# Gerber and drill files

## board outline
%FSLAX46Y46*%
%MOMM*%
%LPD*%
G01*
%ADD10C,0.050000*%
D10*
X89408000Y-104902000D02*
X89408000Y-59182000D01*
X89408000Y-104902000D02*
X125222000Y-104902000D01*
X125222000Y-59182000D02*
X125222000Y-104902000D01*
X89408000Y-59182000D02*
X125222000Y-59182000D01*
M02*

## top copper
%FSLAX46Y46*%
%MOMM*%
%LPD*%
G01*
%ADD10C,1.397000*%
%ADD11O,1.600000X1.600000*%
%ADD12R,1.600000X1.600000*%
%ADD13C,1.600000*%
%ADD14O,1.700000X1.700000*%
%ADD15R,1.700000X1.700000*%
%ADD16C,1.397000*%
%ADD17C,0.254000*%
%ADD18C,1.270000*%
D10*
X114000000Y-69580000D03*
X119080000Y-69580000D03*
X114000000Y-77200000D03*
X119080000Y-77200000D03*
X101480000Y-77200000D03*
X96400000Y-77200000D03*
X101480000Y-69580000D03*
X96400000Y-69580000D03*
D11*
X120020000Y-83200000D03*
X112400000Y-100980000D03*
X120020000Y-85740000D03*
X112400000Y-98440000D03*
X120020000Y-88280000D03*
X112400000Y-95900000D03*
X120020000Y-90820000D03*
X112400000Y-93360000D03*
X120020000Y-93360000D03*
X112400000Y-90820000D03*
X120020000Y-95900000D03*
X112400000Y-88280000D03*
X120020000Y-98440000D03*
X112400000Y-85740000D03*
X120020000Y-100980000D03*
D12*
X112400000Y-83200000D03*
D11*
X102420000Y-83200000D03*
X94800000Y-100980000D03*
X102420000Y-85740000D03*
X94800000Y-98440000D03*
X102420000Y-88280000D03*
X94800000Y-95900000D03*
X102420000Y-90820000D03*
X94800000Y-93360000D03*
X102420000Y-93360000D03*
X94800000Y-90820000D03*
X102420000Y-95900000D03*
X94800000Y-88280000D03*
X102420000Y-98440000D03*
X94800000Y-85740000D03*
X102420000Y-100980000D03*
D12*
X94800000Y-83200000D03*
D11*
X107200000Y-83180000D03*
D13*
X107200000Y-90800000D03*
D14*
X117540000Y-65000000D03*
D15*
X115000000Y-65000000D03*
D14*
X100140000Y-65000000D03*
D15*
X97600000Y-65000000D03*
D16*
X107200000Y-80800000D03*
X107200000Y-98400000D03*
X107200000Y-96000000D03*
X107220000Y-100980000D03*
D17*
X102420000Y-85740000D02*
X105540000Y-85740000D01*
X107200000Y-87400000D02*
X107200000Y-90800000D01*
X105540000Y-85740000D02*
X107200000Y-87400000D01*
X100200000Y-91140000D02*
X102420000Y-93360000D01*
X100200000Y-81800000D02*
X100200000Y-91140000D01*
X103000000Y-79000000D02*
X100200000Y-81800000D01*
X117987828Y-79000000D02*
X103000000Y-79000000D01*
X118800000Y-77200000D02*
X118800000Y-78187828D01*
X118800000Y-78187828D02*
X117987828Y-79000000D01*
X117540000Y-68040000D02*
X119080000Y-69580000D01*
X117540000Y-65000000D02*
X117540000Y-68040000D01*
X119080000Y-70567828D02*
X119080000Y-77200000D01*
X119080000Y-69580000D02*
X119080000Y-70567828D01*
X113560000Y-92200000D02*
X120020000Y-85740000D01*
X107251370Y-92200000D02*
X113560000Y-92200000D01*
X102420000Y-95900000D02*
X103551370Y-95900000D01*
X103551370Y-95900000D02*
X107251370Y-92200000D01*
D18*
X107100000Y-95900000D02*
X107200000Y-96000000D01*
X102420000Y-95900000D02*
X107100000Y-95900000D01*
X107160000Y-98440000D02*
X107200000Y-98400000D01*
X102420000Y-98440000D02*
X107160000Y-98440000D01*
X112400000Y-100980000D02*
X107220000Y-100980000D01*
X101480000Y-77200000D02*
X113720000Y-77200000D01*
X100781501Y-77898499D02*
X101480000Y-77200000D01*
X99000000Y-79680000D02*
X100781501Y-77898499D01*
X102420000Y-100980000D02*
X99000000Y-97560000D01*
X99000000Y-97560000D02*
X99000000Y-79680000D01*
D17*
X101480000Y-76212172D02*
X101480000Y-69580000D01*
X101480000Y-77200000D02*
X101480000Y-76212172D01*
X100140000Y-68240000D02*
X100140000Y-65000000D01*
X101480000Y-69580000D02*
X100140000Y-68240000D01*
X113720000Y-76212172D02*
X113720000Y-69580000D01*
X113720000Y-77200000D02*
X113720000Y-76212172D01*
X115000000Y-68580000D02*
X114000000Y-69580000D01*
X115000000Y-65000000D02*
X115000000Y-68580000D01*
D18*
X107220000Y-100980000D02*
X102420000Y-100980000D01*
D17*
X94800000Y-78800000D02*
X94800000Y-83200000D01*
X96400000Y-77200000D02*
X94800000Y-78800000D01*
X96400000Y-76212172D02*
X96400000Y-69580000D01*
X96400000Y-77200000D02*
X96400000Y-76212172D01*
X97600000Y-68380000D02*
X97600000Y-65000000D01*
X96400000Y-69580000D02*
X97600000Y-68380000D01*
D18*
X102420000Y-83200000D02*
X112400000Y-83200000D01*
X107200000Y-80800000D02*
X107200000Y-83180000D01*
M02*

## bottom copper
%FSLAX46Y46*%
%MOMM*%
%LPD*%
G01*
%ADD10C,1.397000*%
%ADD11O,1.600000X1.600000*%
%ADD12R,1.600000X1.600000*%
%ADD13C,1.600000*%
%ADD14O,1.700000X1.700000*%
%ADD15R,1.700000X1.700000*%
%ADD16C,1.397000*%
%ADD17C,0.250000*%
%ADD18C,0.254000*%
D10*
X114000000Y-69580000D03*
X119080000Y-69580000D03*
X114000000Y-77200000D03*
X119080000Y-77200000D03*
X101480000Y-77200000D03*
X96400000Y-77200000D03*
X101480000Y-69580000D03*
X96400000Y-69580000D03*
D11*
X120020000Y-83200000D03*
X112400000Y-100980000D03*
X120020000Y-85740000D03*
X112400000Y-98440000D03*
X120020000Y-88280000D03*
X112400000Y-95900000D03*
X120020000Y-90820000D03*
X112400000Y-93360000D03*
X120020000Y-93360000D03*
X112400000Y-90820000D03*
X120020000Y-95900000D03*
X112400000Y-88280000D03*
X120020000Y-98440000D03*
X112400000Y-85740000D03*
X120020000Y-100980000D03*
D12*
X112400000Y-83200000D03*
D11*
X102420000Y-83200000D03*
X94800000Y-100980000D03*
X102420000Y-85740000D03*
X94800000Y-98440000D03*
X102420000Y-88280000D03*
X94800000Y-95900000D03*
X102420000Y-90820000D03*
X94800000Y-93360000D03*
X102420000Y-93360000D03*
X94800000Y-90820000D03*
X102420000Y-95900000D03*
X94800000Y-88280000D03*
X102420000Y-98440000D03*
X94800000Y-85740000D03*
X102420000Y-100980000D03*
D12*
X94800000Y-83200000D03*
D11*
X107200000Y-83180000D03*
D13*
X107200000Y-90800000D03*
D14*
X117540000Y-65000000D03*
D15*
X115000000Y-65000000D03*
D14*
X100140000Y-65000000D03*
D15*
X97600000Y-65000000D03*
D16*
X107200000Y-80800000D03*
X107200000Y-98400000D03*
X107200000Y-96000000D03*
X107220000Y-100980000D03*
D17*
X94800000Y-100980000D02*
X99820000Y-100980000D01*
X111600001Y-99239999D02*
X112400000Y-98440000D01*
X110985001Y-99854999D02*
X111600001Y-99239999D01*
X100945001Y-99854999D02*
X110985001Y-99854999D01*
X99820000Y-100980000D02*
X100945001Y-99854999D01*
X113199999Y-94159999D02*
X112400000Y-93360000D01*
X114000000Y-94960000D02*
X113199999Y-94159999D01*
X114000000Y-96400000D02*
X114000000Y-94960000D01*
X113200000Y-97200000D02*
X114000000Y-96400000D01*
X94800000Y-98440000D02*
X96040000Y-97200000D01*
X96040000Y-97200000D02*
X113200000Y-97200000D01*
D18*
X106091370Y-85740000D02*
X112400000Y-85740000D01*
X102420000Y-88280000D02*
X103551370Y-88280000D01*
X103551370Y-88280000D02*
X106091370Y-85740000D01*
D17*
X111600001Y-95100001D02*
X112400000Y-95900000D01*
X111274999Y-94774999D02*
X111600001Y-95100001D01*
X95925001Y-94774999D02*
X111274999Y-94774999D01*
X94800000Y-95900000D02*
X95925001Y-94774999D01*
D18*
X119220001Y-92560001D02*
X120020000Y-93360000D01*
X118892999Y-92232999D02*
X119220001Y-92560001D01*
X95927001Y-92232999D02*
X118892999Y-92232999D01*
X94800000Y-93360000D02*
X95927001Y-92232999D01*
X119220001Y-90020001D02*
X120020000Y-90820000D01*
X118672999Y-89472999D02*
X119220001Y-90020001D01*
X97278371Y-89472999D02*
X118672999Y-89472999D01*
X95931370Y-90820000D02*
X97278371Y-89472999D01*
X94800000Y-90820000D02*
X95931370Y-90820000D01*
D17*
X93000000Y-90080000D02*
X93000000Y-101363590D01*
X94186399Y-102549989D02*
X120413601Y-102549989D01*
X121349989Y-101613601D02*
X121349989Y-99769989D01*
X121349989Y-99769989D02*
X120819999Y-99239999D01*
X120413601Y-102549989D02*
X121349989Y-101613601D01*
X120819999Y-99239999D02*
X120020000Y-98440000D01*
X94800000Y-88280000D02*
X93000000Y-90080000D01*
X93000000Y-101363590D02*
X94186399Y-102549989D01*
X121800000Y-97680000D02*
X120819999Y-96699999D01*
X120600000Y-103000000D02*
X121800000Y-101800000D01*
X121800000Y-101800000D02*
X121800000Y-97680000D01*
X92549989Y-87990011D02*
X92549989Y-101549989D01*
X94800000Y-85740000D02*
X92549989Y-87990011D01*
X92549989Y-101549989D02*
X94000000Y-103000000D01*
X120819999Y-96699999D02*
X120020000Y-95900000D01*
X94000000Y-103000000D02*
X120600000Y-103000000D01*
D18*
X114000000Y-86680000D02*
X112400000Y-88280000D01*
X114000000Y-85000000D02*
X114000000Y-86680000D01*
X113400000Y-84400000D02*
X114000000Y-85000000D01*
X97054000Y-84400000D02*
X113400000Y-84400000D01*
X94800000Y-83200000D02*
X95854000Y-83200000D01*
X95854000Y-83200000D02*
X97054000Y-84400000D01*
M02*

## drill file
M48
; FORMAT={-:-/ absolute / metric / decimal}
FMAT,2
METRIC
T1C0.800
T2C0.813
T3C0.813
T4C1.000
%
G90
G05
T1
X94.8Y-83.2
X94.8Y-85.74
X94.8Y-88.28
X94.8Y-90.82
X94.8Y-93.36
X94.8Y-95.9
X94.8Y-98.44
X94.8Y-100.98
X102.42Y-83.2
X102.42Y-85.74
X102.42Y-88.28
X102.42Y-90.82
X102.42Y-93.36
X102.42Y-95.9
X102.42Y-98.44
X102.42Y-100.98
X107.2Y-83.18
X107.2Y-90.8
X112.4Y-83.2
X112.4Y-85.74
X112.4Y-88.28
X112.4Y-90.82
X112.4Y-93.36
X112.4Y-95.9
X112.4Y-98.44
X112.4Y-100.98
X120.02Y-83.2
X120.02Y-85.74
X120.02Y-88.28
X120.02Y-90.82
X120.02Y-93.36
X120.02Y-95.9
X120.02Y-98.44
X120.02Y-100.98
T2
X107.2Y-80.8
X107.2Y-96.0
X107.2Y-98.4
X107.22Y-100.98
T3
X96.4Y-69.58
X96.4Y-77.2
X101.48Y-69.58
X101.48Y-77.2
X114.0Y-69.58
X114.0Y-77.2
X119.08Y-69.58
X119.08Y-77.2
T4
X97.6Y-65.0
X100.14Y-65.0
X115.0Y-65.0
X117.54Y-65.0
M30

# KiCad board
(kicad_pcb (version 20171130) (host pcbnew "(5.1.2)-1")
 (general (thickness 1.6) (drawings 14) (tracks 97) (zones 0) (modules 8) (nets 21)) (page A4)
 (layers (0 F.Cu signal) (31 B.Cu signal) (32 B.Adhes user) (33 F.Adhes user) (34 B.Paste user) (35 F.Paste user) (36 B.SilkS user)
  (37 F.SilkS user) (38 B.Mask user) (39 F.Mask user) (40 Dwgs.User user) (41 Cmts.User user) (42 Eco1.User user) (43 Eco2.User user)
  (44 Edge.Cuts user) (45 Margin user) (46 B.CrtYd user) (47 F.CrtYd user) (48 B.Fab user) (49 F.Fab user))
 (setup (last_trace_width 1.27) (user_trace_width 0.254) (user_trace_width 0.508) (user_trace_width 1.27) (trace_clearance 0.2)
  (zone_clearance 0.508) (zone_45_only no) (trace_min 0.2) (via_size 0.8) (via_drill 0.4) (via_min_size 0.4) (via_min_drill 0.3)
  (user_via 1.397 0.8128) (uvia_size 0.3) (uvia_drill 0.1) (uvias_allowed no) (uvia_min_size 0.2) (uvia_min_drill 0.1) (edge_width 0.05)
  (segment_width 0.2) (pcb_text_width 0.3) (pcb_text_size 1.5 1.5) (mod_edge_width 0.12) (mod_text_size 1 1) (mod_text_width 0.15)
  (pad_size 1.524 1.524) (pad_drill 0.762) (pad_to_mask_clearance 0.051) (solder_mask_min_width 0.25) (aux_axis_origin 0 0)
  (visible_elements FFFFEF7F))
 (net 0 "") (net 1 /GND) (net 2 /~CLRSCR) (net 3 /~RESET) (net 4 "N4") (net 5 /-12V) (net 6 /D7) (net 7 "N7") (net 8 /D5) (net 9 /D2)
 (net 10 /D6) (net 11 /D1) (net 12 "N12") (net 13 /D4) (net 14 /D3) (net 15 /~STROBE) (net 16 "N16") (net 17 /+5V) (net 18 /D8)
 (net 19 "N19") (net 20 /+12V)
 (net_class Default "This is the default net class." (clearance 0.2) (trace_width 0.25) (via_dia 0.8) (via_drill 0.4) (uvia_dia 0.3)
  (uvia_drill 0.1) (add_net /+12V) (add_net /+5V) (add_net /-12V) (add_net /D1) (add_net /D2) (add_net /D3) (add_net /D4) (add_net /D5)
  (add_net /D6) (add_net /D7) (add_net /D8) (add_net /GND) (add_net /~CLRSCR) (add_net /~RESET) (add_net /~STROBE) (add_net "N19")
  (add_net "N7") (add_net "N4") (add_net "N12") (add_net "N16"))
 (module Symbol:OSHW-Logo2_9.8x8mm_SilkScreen (layer F.Cu) (at 107.2388 71.1454 90)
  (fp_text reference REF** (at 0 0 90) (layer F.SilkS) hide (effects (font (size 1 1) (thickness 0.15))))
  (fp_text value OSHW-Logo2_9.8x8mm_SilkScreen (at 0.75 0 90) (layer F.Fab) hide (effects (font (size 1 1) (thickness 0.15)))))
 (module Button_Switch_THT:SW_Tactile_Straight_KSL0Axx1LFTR (layer F.Cu) (at 114 77.2 90)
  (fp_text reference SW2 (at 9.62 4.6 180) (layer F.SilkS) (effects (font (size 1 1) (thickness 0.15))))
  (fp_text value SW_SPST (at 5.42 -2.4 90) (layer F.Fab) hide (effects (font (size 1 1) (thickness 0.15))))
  (pad 1 thru_hole circle (at 7.62 0 90) (size 1.397 1.397) (drill 0.8128) (layers *.Cu *.Mask) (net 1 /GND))
  (pad 2 thru_hole circle (at 7.62 5.08 90) (size 1.397 1.397) (drill 0.8128) (layers *.Cu *.Mask) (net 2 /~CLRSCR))
  (pad 1 thru_hole circle (at 0 0 90) (size 1.397 1.397) (drill 0.8128) (layers *.Cu *.Mask) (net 1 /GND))
  (pad 2 thru_hole circle (at 0 5.08 90) (size 1.397 1.397) (drill 0.8128) (layers *.Cu *.Mask) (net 2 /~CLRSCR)))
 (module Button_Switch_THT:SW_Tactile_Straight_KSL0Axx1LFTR (layer F.Cu) (at 96.4 77.2 90)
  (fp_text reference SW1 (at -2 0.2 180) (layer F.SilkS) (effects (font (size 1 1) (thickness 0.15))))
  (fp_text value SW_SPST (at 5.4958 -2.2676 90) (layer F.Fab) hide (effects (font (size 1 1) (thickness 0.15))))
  (pad 2 thru_hole circle (at 0 5.08 90) (size 1.397 1.397) (drill 0.8128) (layers *.Cu *.Mask) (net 1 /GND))
  (pad 1 thru_hole circle (at 0 0 90) (size 1.397 1.397) (drill 0.8128) (layers *.Cu *.Mask) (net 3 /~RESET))
  (pad 2 thru_hole circle (at 7.62 5.08 90) (size 1.397 1.397) (drill 0.8128) (layers *.Cu *.Mask) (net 1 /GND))
  (pad 1 thru_hole circle (at 7.62 0 90) (size 1.397 1.397) (drill 0.8128) (layers *.Cu *.Mask) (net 3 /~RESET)))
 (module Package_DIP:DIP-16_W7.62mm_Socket (layer F.Cu) (at 112.4 83.2)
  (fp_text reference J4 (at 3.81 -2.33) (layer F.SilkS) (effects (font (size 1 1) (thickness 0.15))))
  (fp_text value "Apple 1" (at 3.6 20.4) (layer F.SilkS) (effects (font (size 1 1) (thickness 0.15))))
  (pad 16 thru_hole oval (at 7.62 0) (size 1.6 1.6) (drill 0.8) (layers *.Cu *.Mask) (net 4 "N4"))
  (pad 8 thru_hole oval (at 0 17.78) (size 1.6 1.6) (drill 0.8) (layers *.Cu *.Mask) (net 1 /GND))
  (pad 15 thru_hole oval (at 7.62 2.54) (size 1.6 1.6) (drill 0.8) (layers *.Cu *.Mask) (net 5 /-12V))
  (pad 7 thru_hole oval (at 0 15.24) (size 1.6 1.6) (drill 0.8) (layers *.Cu *.Mask) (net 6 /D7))
  (pad 14 thru_hole oval (at 7.62 5.08) (size 1.6 1.6) (drill 0.8) (layers *.Cu *.Mask) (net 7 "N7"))
  (pad 6 thru_hole oval (at 0 12.7) (size 1.6 1.6) (drill 0.8) (layers *.Cu *.Mask) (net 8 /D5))
  (pad 13 thru_hole oval (at 7.62 7.62) (size 1.6 1.6) (drill 0.8) (layers *.Cu *.Mask) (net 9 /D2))
  (pad 5 thru_hole oval (at 0 10.16) (size 1.6 1.6) (drill 0.8) (layers *.Cu *.Mask) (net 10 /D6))
  (pad 12 thru_hole oval (at 7.62 10.16) (size 1.6 1.6) (drill 0.8) (layers *.Cu *.Mask) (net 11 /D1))
  (pad 4 thru_hole oval (at 0 7.62) (size 1.6 1.6) (drill 0.8) (layers *.Cu *.Mask) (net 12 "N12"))
  (pad 11 thru_hole oval (at 7.62 12.7) (size 1.6 1.6) (drill 0.8) (layers *.Cu *.Mask) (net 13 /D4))
  (pad 3 thru_hole oval (at 0 5.08) (size 1.6 1.6) (drill 0.8) (layers *.Cu *.Mask) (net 3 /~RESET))
  (pad 10 thru_hole oval (at 7.62 15.24) (size 1.6 1.6) (drill 0.8) (layers *.Cu *.Mask) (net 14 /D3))
  (pad 2 thru_hole oval (at 0 2.54) (size 1.6 1.6) (drill 0.8) (layers *.Cu *.Mask) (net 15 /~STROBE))
  (pad 9 thru_hole oval (at 7.62 17.78) (size 1.6 1.6) (drill 0.8) (layers *.Cu *.Mask) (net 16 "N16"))
  (pad 1 thru_hole rect (at 0 0) (size 1.6 1.6) (drill 0.8) (layers *.Cu *.Mask) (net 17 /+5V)))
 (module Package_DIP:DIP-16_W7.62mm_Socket (layer F.Cu) (at 94.8 83.2)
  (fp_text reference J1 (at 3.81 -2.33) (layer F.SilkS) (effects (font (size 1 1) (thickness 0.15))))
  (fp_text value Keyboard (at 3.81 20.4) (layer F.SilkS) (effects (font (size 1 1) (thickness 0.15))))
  (pad 16 thru_hole oval (at 7.62 0) (size 1.6 1.6) (drill 0.8) (layers *.Cu *.Mask) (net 17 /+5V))
  (pad 8 thru_hole oval (at 0 17.78) (size 1.6 1.6) (drill 0.8) (layers *.Cu *.Mask) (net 6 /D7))
  (pad 15 thru_hole oval (at 7.62 2.54) (size 1.6 1.6) (drill 0.8) (layers *.Cu *.Mask) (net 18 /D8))
  (pad 7 thru_hole oval (at 0 15.24) (size 1.6 1.6) (drill 0.8) (layers *.Cu *.Mask) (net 10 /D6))
  (pad 14 thru_hole oval (at 7.62 5.08) (size 1.6 1.6) (drill 0.8) (layers *.Cu *.Mask) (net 15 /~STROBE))
  (pad 6 thru_hole oval (at 0 12.7) (size 1.6 1.6) (drill 0.8) (layers *.Cu *.Mask) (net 8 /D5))
  (pad 13 thru_hole oval (at 7.62 7.62) (size 1.6 1.6) (drill 0.8) (layers *.Cu *.Mask) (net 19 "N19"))
  (pad 5 thru_hole oval (at 0 10.16) (size 1.6 1.6) (drill 0.8) (layers *.Cu *.Mask) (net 11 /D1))
  (pad 12 thru_hole oval (at 7.62 10.16) (size 1.6 1.6) (drill 0.8) (layers *.Cu *.Mask) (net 2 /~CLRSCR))
  (pad 4 thru_hole oval (at 0 7.62) (size 1.6 1.6) (drill 0.8) (layers *.Cu *.Mask) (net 9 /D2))
  (pad 11 thru_hole oval (at 7.62 12.7) (size 1.6 1.6) (drill 0.8) (layers *.Cu *.Mask) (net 5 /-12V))
  (pad 3 thru_hole oval (at 0 5.08) (size 1.6 1.6) (drill 0.8) (layers *.Cu *.Mask) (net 14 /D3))
  (pad 10 thru_hole oval (at 7.62 15.24) (size 1.6 1.6) (drill 0.8) (layers *.Cu *.Mask) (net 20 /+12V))
  (pad 2 thru_hole oval (at 0 2.54) (size 1.6 1.6) (drill 0.8) (layers *.Cu *.Mask) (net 13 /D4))
  (pad 9 thru_hole oval (at 7.62 17.78) (size 1.6 1.6) (drill 0.8) (layers *.Cu *.Mask) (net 1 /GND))
  (pad 1 thru_hole rect (at 0 0) (size 1.6 1.6) (drill 0.8) (layers *.Cu *.Mask) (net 3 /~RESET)))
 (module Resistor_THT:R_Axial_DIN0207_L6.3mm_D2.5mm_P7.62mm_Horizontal (layer F.Cu) (at 107.2 90.8 90)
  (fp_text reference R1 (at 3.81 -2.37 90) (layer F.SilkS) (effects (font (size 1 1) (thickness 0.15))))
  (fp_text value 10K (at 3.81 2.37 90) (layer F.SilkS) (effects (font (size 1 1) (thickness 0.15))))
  (pad 2 thru_hole oval (at 7.62 0 90) (size 1.6 1.6) (drill 0.8) (layers *.Cu *.Mask) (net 17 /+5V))
  (pad 1 thru_hole circle (at 0 0 90) (size 1.6 1.6) (drill 0.8) (layers *.Cu *.Mask) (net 18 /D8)))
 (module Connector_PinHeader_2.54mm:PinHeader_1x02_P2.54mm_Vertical (layer F.Cu) (at 115 65 90)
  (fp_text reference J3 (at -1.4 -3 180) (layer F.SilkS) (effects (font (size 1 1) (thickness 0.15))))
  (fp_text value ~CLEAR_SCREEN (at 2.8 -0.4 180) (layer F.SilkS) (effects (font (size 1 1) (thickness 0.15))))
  (pad 2 thru_hole oval (at 0 2.54 90) (size 1.7 1.7) (drill 1) (layers *.Cu *.Mask) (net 2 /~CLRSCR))
  (pad 1 thru_hole rect (at 0 0 90) (size 1.7 1.7) (drill 1) (layers *.Cu *.Mask) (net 1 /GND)))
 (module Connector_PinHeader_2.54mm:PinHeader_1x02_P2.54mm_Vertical (layer F.Cu) (at 97.6 65 90)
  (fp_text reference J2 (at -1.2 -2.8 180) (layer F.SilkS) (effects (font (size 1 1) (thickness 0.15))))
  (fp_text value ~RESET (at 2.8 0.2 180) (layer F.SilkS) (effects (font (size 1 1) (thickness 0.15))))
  (pad 2 thru_hole oval (at 0 2.54 90) (size 1.7 1.7) (drill 1) (layers *.Cu *.Mask) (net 1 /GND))
  (pad 1 thru_hole rect (at 0 0 90) (size 1.7 1.7) (drill 1) (layers *.Cu *.Mask) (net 3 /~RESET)))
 (gr_line (start 89.408 104.902) (end 89.408 59.182) (layer Edge.Cuts) (width 0.05))
 (gr_line (start 89.408 104.902) (end 125.222 104.902) (layer Edge.Cuts) (width 0.05))
 (gr_line (start 125.222 59.182) (end 125.222 104.902) (layer Edge.Cuts) (width 0.05))
 (gr_line (start 89.408 59.182) (end 125.222 59.182) (layer Edge.Cuts) (width 0.05))
 (via (at 107.2 80.8) (size 1.397) (drill 0.8128) (layers F.Cu B.Cu) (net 17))
 (via (at 107.2 98.4) (size 1.397) (drill 0.8128) (layers F.Cu B.Cu) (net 20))
 (via (at 107.2 96) (size 1.397) (drill 0.8128) (layers F.Cu B.Cu) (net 5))
 (segment (start 94.8 100.98) (end 99.82 100.98) (width 0.25) (layer B.Cu) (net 6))
 (segment (start 111.600001 99.239999) (end 112.4 98.44) (width 0.25) (layer B.Cu) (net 6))
 (segment (start 110.985001 99.854999) (end 111.600001 99.239999) (width 0.25) (layer B.Cu) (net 6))
 (segment (start 100.945001 99.854999) (end 110.985001 99.854999) (width 0.25) (layer B.Cu) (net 6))
 (segment (start 99.82 100.98) (end 100.945001 99.854999) (width 0.25) (layer B.Cu) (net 6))
 (segment (start 102.42 85.74) (end 105.54 85.74) (width 0.254) (layer F.Cu) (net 18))
 (segment (start 107.2 87.4) (end 107.2 90.8) (width 0.254) (layer F.Cu) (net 18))
 (segment (start 105.54 85.74) (end 107.2 87.4) (width 0.254) (layer F.Cu) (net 18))
 (segment (start 113.199999 94.159999) (end 112.4 93.36) (width 0.25) (layer B.Cu) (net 10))
 (segment (start 114 94.96) (end 113.199999 94.159999) (width 0.25) (layer B.Cu) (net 10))
 (segment (start 114 96.4) (end 114 94.96) (width 0.25) (layer B.Cu) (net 10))
 (segment (start 113.2 97.2) (end 114 96.4) (width 0.25) (layer B.Cu) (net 10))
 (segment (start 94.8 98.44) (end 96.04 97.2) (width 0.25) (layer B.Cu) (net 10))
 (segment (start 96.04 97.2) (end 113.2 97.2) (width 0.25) (layer B.Cu) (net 10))
 (segment (start 106.09137 85.74) (end 112.4 85.74) (width 0.254) (layer B.Cu) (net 15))
 (segment (start 102.42 88.28) (end 103.55137 88.28) (width 0.254) (layer B.Cu) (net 15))
 (segment (start 103.55137 88.28) (end 106.09137 85.74) (width 0.254) (layer B.Cu) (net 15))
 (segment (start 111.600001 95.100001) (end 112.4 95.9) (width 0.25) (layer B.Cu) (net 8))
 (segment (start 111.274999 94.774999) (end 111.600001 95.100001) (width 0.25) (layer B.Cu) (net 8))
 (segment (start 95.925001 94.774999) (end 111.274999 94.774999) (width 0.25) (layer B.Cu) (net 8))
 (segment (start 94.8 95.9) (end 95.925001 94.774999) (width 0.25) (layer B.Cu) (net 8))
 (segment (start 119.220001 92.560001) (end 120.02 93.36) (width 0.254) (layer B.Cu) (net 11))
 (segment (start 118.892999 92.232999) (end 119.220001 92.560001) (width 0.254) (layer B.Cu) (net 11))
 (segment (start 95.927001 92.232999) (end 118.892999 92.232999) (width 0.254) (layer B.Cu) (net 11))
 (segment (start 94.8 93.36) (end 95.927001 92.232999) (width 0.254) (layer B.Cu) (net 11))
 (segment (start 100.2 91.14) (end 102.42 93.36) (width 0.254) (layer F.Cu) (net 2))
 (segment (start 100.2 81.8) (end 100.2 91.14) (width 0.254) (layer F.Cu) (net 2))
 (segment (start 103 79) (end 100.2 81.8) (width 0.254) (layer F.Cu) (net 2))
 (segment (start 117.987828 79) (end 103 79) (width 0.254) (layer F.Cu) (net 2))
 (segment (start 118.8 77.2) (end 118.8 78.187828) (width 0.254) (layer F.Cu) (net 2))
 (segment (start 118.8 78.187828) (end 117.987828 79) (width 0.254) (layer F.Cu) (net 2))
 (segment (start 117.54 68.04) (end 119.08 69.58) (width 0.254) (layer F.Cu) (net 2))
 (segment (start 117.54 65) (end 117.54 68.04) (width 0.254) (layer F.Cu) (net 2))
 (segment (start 119.08 70.567828) (end 119.08 77.2) (width 0.254) (layer F.Cu) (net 2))
 (segment (start 119.08 69.58) (end 119.08 70.567828) (width 0.254) (layer F.Cu) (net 2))
 (segment (start 119.220001 90.020001) (end 120.02 90.82) (width 0.254) (layer B.Cu) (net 9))
 (segment (start 118.672999 89.472999) (end 119.220001 90.020001) (width 0.254) (layer B.Cu) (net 9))
 (segment (start 97.278371 89.472999) (end 118.672999 89.472999) (width 0.254) (layer B.Cu) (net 9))
 (segment (start 95.93137 90.82) (end 97.278371 89.472999) (width 0.254) (layer B.Cu) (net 9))
 (segment (start 94.8 90.82) (end 95.93137 90.82) (width 0.254) (layer B.Cu) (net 9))
 (segment (start 113.56 92.2) (end 120.02 85.74) (width 0.254) (layer F.Cu) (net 5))
 (segment (start 107.25137 92.2) (end 113.56 92.2) (width 0.254) (layer F.Cu) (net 5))
 (segment (start 102.42 95.9) (end 103.55137 95.9) (width 0.254) (layer F.Cu) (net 5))
 (segment (start 103.55137 95.9) (end 107.25137 92.2) (width 0.254) (layer F.Cu) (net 5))
 (segment (start 107.1 95.9) (end 107.2 96) (width 1.27) (layer F.Cu) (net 5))
 (segment (start 102.42 95.9) (end 107.1 95.9) (width 1.27) (layer F.Cu) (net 5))
 (segment (start 93 90.08) (end 93 101.36359) (width 0.25) (layer B.Cu) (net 14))
 (segment (start 94.186399 102.549989) (end 120.413601 102.549989) (width 0.25) (layer B.Cu) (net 14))
 (segment (start 121.349989 101.613601) (end 121.349989 99.769989) (width 0.25) (layer B.Cu) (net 14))
 (segment (start 121.349989 99.769989) (end 120.819999 99.239999) (width 0.25) (layer B.Cu) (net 14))
 (segment (start 120.413601 102.549989) (end 121.349989 101.613601) (width 0.25) (layer B.Cu) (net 14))
 (segment (start 120.819999 99.239999) (end 120.02 98.44) (width 0.25) (layer B.Cu) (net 14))
 (segment (start 94.8 88.28) (end 93 90.08) (width 0.25) (layer B.Cu) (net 14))
 (segment (start 93 101.36359) (end 94.186399 102.549989) (width 0.25) (layer B.Cu) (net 14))
 (segment (start 107.16 98.44) (end 107.2 98.4) (width 1.27) (layer F.Cu) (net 20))
 (segment (start 102.42 98.44) (end 107.16 98.44) (width 1.27) (layer F.Cu) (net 20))
 (segment (start 121.8 97.68) (end 120.819999 96.699999) (width 0.25) (layer B.Cu) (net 13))
 (segment (start 120.6 103) (end 121.8 101.8) (width 0.25) (layer B.Cu) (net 13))
 (segment (start 121.8 101.8) (end 121.8 97.68) (width 0.25) (layer B.Cu) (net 13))
 (segment (start 92.549989 87.990011) (end 92.549989 101.549989) (width 0.25) (layer B.Cu) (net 13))
 (segment (start 94.8 85.74) (end 92.549989 87.990011) (width 0.25) (layer B.Cu) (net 13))
 (segment (start 92.549989 101.549989) (end 94 103) (width 0.25) (layer B.Cu) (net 13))
 (segment (start 120.819999 96.699999) (end 120.02 95.9) (width 0.25) (layer B.Cu) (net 13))
 (segment (start 94 103) (end 120.6 103) (width 0.25) (layer B.Cu) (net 13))
 (segment (start 112.4 100.98) (end 107.22 100.98) (width 1.27) (layer F.Cu) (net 1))
 (segment (start 101.48 77.2) (end 113.72 77.2) (width 1.27) (layer F.Cu) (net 1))
 (segment (start 100.781501 77.898499) (end 101.48 77.2) (width 1.27) (layer F.Cu) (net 1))
 (segment (start 99 79.68) (end 100.781501 77.898499) (width 1.27) (layer F.Cu) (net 1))
 (segment (start 102.42 100.98) (end 99 97.56) (width 1.27) (layer F.Cu) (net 1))
 (segment (start 99 97.56) (end 99 79.68) (width 1.27) (layer F.Cu) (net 1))
 (segment (start 101.48 76.212172) (end 101.48 69.58) (width 0.254) (layer F.Cu) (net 1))
 (segment (start 101.48 77.2) (end 101.48 76.212172) (width 0.254) (layer F.Cu) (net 1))
 (segment (start 100.14 68.24) (end 100.14 65) (width 0.254) (layer F.Cu) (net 1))
 (segment (start 101.48 69.58) (end 100.14 68.24) (width 0.254) (layer F.Cu) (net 1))
 (segment (start 113.72 76.212172) (end 113.72 69.58) (width 0.254) (layer F.Cu) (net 1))
 (segment (start 113.72 77.2) (end 113.72 76.212172) (width 0.254) (layer F.Cu) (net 1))
 (segment (start 115 68.58) (end 114 69.58) (width 0.254) (layer F.Cu) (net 1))
 (segment (start 115 65) (end 115 68.58) (width 0.254) (layer F.Cu) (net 1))
 (segment (start 107.22 100.98) (end 102.42 100.98) (width 1.27) (layer F.Cu) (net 1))
 (via (at 107.22 100.98) (size 1.397) (drill 0.8128) (layers F.Cu B.Cu) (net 1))
 (segment (start 114 86.68) (end 112.4 88.28) (width 0.254) (layer B.Cu) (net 3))
 (segment (start 114 85) (end 114 86.68) (width 0.254) (layer B.Cu) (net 3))
 (segment (start 113.4 84.4) (end 114 85) (width 0.254) (layer B.Cu) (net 3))
 (segment (start 97.054 84.4) (end 113.4 84.4) (width 0.254) (layer B.Cu) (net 3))
 (segment (start 94.8 83.2) (end 95.854 83.2) (width 0.254) (layer B.Cu) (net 3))
 (segment (start 95.854 83.2) (end 97.054 84.4) (width 0.254) (layer B.Cu) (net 3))
 (segment (start 94.8 78.8) (end 94.8 83.2) (width 0.254) (layer F.Cu) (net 3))
 (segment (start 96.4 77.2) (end 94.8 78.8) (width 0.254) (layer F.Cu) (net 3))
 (segment (start 96.4 76.212172) (end 96.4 69.58) (width 0.254) (layer F.Cu) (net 3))
 (segment (start 96.4 77.2) (end 96.4 76.212172) (width 0.254) (layer F.Cu) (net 3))
 (segment (start 97.6 68.38) (end 97.6 65) (width 0.254) (layer F.Cu) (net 3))
 (segment (start 96.4 69.58) (end 97.6 68.38) (width 0.254) (layer F.Cu) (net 3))
 (segment (start 102.42 83.2) (end 112.4 83.2) (width 1.27) (layer F.Cu) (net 17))
 (segment (start 107.2 80.8) (end 107.2 83.18) (width 1.27) (layer F.Cu) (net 17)))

